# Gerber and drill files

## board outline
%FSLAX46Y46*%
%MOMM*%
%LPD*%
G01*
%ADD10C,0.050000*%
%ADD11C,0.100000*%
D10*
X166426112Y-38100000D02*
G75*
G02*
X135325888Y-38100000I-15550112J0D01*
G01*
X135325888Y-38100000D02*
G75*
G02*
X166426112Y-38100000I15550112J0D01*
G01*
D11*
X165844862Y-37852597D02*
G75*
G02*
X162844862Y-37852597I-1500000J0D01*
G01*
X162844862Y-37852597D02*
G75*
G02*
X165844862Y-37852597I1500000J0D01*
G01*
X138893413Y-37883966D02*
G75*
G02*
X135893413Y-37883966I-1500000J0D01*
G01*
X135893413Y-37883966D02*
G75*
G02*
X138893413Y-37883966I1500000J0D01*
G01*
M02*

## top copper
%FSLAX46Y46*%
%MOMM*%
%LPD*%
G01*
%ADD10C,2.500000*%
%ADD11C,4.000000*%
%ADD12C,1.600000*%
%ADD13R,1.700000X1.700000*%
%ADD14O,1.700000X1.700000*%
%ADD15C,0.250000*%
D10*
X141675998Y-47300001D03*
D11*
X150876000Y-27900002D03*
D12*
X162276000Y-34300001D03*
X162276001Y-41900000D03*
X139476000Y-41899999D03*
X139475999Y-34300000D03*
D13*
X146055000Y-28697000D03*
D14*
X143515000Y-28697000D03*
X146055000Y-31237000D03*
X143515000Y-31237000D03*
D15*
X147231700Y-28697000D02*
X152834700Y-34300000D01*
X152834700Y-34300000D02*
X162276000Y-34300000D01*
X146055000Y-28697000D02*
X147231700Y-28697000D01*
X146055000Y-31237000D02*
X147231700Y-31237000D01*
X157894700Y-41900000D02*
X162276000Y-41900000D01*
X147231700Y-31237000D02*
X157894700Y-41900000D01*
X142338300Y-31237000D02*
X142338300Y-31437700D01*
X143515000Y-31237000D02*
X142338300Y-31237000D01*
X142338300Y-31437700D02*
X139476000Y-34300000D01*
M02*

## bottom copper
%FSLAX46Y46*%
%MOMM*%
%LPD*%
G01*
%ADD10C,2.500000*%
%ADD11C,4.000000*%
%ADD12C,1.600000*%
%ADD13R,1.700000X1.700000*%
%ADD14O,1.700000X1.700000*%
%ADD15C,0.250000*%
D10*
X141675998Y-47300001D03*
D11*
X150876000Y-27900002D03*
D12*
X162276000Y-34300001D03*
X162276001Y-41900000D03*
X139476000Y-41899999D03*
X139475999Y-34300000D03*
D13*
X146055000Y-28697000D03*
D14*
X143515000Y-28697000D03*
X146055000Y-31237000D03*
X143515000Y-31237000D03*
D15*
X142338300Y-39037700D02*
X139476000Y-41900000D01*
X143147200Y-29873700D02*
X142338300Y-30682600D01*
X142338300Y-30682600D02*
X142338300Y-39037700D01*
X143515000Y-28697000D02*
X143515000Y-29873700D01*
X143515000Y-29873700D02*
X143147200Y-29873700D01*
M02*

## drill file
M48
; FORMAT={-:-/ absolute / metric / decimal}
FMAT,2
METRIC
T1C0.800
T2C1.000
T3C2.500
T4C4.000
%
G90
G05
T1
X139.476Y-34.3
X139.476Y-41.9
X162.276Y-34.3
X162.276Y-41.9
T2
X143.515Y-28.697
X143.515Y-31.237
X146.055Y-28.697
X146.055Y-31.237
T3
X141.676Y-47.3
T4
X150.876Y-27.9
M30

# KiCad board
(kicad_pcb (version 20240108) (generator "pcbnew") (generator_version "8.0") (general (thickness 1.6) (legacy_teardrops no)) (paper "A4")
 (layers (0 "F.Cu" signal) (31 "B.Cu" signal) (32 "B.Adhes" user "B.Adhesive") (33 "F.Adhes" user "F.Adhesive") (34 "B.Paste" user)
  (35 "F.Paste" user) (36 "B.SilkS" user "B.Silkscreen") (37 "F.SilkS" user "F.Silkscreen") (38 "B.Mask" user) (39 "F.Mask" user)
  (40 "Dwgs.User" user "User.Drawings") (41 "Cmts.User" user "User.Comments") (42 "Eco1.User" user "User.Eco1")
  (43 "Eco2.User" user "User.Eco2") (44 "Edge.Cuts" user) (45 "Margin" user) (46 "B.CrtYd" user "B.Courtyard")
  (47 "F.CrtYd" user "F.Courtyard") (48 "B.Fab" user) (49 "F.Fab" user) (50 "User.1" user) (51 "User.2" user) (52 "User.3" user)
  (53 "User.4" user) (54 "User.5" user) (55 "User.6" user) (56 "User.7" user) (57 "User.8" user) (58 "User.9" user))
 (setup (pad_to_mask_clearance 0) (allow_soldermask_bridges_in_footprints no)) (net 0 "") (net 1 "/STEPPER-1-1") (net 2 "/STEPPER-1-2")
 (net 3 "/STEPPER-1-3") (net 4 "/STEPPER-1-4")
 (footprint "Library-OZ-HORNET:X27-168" (layer "F.Cu") (at 150.876 38.1)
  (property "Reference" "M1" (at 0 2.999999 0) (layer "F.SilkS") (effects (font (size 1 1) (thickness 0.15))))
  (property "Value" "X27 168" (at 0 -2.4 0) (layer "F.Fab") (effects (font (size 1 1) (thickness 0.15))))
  (pad "" thru_hole circle (at -9.200002 9.200001) (size 2.5 2.5) (drill 2.5) (layers "*.Cu" "*.Mask") (remove_unused_layers no))
  (pad "" thru_hole circle (at 0 -10.199998) (size 4 4) (drill 4) (layers "*.Cu" "*.Mask") (remove_unused_layers no))
  (pad "1" thru_hole circle (at 11.4 -3.799999) (size 1.6 1.6) (drill 0.8) (layers "*.Cu" "*.Mask") (remove_unused_layers no)
   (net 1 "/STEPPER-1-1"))
  (pad "2" thru_hole circle (at 11.400001 3.8) (size 1.6 1.6) (drill 0.8) (layers "*.Cu" "*.Mask") (remove_unused_layers no)
   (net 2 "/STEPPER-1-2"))
  (pad "3" thru_hole circle (at -11.4 3.799999) (size 1.6 1.6) (drill 0.8) (layers "*.Cu" "*.Mask") (remove_unused_layers no)
   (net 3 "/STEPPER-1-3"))
  (pad "4" thru_hole circle (at -11.400001 -3.8) (size 1.6 1.6) (drill 0.8) (layers "*.Cu" "*.Mask") (remove_unused_layers no)
   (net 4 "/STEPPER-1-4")))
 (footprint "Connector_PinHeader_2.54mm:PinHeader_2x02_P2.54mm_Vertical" (layer "B.Cu") (at 146.055 28.697 180)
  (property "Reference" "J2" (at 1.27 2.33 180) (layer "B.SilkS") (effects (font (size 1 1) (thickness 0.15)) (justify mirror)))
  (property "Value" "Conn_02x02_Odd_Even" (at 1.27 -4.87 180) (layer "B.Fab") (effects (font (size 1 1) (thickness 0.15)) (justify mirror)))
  (pad "1" thru_hole rect (at 0 0 180) (size 1.7 1.7) (drill 1) (layers "*.Cu" "*.Mask") (remove_unused_layers no) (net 1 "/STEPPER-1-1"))
  (pad "2" thru_hole oval (at 2.54 0 180) (size 1.7 1.7) (drill 1) (layers "*.Cu" "*.Mask") (remove_unused_layers no) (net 3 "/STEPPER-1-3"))
  (pad "3" thru_hole oval (at 0 -2.54 180) (size 1.7 1.7) (drill 1) (layers "*.Cu" "*.Mask") (remove_unused_layers no)
   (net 2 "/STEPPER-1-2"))
  (pad "4" thru_hole oval (at 2.54 -2.54 180) (size 1.7 1.7) (drill 1) (layers "*.Cu" "*.Mask") (remove_unused_layers no)
   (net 4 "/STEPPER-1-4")))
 (gr_circle (center 150.876 38.1) (end 166.426112 38.1) (stroke (width 0.05) (type default)) (fill none) (layer "Edge.Cuts"))
 (gr_circle (center 164.344862 37.852597) (end 165.844862 37.852597) (stroke (width 0.1) (type default)) (fill none) (layer "Edge.Cuts"))
 (gr_circle (center 137.393413 37.883966) (end 138.893413 37.883966) (stroke (width 0.1) (type default)) (fill none) (layer "Edge.Cuts"))
 (segment (start 147.2317 28.697) (end 152.8347 34.3) (width 0.25) (layer "F.Cu") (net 1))
 (segment (start 152.8347 34.3) (end 162.276 34.3) (width 0.25) (layer "F.Cu") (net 1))
 (segment (start 146.055 28.697) (end 147.2317 28.697) (width 0.25) (layer "F.Cu") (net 1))
 (segment (start 146.055 31.237) (end 147.2317 31.237) (width 0.25) (layer "F.Cu") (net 2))
 (segment (start 157.8947 41.9) (end 162.276 41.9) (width 0.25) (layer "F.Cu") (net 2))
 (segment (start 147.2317 31.237) (end 157.8947 41.9) (width 0.25) (layer "F.Cu") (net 2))
 (segment (start 142.3383 39.0377) (end 139.476 41.9) (width 0.25) (layer "B.Cu") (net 3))
 (segment (start 143.1472 29.8737) (end 142.3383 30.6826) (width 0.25) (layer "B.Cu") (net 3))
 (segment (start 142.3383 30.6826) (end 142.3383 39.0377) (width 0.25) (layer "B.Cu") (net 3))
 (segment (start 143.515 28.697) (end 143.515 29.8737) (width 0.25) (layer "B.Cu") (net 3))
 (segment (start 143.515 29.8737) (end 143.1472 29.8737) (width 0.25) (layer "B.Cu") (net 3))
 (segment (start 142.3383 31.237) (end 142.3383 31.4377) (width 0.25) (layer "F.Cu") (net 4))
 (segment (start 143.515 31.237) (end 142.3383 31.237) (width 0.25) (layer "F.Cu") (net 4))
 (segment (start 142.3383 31.4377) (end 139.476 34.3) (width 0.25) (layer "F.Cu") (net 4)))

